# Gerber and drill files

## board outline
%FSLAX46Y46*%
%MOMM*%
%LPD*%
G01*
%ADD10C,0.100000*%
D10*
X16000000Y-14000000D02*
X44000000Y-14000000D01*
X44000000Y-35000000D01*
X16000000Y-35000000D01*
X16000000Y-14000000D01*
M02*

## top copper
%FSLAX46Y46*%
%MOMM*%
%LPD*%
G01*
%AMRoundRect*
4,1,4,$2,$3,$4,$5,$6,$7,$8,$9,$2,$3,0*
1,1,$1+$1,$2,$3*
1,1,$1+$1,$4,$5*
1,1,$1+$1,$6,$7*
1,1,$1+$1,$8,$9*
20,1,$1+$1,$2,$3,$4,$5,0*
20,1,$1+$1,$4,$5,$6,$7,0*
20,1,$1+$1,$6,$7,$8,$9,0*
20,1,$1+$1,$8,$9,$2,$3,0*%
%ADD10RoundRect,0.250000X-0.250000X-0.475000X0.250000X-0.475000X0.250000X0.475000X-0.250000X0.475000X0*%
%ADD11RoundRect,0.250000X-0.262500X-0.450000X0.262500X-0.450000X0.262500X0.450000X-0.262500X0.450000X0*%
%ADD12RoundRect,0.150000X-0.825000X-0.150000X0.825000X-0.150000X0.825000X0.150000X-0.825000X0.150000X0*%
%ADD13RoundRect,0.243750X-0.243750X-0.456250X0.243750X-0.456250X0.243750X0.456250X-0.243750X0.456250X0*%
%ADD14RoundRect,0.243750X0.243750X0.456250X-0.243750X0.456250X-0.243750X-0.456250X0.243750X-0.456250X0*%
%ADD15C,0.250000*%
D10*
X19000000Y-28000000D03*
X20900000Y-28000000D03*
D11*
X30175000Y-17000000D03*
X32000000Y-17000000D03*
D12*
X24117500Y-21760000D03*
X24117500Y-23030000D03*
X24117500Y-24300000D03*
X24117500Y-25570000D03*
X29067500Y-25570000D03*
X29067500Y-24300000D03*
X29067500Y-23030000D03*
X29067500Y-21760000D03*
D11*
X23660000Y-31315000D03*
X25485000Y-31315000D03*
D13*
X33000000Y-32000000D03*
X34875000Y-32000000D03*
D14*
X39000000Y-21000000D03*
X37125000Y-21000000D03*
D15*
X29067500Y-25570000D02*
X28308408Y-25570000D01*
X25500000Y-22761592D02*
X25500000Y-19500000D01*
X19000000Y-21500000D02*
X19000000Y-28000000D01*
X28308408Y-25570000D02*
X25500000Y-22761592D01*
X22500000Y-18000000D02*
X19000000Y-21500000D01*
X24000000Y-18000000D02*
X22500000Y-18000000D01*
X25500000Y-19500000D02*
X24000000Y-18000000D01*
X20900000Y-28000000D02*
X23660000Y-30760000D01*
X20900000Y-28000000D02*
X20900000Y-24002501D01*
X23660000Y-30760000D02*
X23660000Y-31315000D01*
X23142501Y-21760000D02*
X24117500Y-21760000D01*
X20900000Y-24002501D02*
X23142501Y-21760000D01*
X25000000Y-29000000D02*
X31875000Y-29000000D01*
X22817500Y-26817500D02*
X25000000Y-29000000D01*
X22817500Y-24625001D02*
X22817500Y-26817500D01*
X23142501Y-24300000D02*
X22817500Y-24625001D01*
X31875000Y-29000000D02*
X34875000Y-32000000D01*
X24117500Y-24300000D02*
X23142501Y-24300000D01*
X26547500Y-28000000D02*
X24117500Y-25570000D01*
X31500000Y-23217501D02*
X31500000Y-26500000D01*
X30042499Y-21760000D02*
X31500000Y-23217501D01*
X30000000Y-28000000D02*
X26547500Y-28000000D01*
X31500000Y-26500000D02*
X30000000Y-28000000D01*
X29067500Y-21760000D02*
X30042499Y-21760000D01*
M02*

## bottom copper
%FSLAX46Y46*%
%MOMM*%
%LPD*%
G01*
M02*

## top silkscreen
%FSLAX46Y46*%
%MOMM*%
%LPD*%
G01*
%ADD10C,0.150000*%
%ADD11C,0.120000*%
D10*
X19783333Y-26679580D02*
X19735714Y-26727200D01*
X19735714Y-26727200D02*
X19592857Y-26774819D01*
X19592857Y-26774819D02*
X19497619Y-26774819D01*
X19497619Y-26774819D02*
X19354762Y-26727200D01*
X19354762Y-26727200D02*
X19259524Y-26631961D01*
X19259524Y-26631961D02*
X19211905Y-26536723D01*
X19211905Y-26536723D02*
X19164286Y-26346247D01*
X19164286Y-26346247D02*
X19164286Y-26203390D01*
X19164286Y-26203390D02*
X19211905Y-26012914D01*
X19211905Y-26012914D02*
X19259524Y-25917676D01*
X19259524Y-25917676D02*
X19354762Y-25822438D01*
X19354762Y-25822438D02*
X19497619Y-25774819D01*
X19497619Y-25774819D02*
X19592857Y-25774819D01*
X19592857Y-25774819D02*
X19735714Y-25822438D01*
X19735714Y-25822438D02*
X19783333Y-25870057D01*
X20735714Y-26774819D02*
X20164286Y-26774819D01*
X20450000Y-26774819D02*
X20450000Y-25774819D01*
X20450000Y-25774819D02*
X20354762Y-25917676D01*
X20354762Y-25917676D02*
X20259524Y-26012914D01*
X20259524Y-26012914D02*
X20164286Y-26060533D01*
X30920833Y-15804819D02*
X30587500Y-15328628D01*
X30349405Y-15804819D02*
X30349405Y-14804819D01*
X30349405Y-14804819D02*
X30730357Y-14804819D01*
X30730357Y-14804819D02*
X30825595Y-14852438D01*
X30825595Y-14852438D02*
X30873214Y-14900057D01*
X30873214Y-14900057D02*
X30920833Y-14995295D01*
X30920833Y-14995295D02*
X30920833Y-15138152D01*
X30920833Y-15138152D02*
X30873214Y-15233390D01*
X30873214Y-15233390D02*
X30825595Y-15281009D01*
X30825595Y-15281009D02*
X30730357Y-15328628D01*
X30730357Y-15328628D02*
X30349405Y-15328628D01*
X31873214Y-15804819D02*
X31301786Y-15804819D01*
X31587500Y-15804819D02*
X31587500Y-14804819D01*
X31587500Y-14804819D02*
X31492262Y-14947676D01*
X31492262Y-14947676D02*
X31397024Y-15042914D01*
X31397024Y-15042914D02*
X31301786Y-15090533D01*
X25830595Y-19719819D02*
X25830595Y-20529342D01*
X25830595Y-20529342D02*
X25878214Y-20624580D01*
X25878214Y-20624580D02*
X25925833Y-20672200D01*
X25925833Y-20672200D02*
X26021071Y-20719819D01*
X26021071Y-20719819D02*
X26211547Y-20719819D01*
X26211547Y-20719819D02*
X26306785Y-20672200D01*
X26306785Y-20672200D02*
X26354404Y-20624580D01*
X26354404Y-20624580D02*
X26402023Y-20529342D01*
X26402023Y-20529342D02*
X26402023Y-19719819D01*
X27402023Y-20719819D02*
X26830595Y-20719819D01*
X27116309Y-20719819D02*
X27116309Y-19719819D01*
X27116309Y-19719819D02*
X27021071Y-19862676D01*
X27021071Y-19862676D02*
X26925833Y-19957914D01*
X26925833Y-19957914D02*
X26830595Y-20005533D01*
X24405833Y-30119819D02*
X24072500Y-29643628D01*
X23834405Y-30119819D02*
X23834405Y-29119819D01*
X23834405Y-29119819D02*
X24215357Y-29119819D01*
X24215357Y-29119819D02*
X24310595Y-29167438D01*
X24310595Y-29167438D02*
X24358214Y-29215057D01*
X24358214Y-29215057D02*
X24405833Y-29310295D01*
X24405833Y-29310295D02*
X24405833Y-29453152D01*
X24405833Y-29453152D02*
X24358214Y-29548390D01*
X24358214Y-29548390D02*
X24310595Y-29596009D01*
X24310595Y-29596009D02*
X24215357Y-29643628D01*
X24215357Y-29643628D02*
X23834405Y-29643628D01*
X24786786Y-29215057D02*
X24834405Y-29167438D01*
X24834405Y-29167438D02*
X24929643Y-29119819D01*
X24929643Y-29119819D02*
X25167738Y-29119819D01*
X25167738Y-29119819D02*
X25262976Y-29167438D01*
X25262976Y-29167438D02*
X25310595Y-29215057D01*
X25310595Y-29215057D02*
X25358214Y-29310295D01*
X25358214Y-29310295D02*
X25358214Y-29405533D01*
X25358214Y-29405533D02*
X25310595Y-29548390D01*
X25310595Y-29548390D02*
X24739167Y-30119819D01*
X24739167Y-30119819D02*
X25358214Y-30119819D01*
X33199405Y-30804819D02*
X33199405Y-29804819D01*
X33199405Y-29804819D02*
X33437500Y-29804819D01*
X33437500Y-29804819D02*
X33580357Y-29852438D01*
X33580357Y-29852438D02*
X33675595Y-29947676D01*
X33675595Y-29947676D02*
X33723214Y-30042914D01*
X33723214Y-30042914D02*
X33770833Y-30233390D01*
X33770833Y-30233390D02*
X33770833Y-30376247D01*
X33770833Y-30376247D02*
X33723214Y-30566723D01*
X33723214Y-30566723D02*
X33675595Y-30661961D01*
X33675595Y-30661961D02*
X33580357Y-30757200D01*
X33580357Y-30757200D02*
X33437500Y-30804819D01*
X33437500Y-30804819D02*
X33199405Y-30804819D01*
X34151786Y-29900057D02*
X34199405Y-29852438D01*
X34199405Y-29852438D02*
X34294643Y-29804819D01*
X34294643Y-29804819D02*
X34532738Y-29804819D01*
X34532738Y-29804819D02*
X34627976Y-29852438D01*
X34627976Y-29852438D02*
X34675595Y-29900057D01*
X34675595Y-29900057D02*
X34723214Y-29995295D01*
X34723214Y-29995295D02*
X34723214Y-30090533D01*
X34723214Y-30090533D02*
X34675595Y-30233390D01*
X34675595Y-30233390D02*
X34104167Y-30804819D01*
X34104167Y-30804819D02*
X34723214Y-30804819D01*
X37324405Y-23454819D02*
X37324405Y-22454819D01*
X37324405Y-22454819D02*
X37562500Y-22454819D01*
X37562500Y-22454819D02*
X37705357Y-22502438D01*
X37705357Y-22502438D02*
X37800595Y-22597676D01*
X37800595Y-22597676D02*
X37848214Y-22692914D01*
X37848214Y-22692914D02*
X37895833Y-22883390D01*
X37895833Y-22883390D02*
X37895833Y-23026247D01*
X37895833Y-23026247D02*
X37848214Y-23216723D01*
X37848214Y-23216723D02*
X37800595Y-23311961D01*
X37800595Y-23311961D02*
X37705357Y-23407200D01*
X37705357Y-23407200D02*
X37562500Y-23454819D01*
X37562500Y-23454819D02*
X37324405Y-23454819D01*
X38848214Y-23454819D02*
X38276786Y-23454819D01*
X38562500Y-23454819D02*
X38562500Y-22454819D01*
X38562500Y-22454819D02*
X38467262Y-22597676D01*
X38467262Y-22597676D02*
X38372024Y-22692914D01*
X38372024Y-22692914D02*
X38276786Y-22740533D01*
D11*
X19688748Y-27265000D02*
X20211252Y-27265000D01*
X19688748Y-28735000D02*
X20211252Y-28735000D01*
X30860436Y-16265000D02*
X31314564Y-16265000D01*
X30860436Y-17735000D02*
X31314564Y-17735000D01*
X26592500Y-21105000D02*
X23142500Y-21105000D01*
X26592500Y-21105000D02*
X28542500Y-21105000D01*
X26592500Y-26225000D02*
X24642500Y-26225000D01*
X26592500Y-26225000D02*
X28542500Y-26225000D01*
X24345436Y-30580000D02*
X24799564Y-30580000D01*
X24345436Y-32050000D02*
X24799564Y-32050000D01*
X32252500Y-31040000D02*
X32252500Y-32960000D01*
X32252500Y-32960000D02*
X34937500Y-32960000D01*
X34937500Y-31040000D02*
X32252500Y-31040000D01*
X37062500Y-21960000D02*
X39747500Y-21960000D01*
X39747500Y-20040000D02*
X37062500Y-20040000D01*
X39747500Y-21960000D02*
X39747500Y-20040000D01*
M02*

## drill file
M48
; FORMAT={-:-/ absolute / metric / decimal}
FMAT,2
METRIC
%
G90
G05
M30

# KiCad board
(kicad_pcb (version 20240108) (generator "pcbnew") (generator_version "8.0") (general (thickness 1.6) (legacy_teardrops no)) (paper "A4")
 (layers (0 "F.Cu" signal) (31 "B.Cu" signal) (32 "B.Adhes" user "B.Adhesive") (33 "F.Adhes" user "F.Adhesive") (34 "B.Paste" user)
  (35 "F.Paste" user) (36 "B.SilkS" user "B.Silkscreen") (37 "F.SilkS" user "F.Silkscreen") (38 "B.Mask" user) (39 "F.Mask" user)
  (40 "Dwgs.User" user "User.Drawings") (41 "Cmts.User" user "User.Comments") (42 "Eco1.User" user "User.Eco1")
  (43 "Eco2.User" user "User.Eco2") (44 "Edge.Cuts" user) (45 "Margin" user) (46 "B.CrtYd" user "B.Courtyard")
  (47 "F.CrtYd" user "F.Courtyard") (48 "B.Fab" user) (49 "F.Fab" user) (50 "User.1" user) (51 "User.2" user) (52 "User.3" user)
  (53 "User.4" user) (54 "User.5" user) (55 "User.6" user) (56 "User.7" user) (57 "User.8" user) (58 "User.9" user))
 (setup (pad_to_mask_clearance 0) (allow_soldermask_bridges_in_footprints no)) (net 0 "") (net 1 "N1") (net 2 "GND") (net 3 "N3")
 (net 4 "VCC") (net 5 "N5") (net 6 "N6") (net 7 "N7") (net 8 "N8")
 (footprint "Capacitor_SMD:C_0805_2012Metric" (layer "F.Cu") (at 19.95 28)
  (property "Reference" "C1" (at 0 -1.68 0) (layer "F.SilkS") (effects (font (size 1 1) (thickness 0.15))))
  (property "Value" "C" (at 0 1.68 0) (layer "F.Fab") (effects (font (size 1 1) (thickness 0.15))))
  (fp_line (start -0.261252 -0.735) (end 0.261252 -0.735) (stroke (width 0.12) (type solid)) (layer "F.SilkS"))
  (fp_line (start -0.261252 0.735) (end 0.261252 0.735) (stroke (width 0.12) (type solid)) (layer "F.SilkS"))
  (pad "1" smd roundrect (at -0.95 0) (size 1 1.45) (layers "F.Cu" "F.Paste" "F.Mask") (roundrect_rratio 0.25) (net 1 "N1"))
  (pad "2" smd roundrect (at 0.95 0) (size 1 1.45) (layers "F.Cu" "F.Paste" "F.Mask") (roundrect_rratio 0.25) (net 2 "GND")))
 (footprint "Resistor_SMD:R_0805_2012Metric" (layer "F.Cu") (at 31.0875 17)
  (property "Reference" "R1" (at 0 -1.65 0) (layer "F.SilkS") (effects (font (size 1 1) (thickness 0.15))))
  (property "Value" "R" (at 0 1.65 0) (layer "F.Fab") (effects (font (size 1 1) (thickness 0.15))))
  (fp_line (start -0.227064 -0.735) (end 0.227064 -0.735) (stroke (width 0.12) (type solid)) (layer "F.SilkS"))
  (fp_line (start -0.227064 0.735) (end 0.227064 0.735) (stroke (width 0.12) (type solid)) (layer "F.SilkS"))
  (pad "1" smd roundrect (at -0.9125 0) (size 1.025 1.4) (layers "F.Cu" "F.Paste" "F.Mask") (roundrect_rratio 0.243902) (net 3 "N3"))
  (pad "2" smd roundrect (at 0.9125 0) (size 1.025 1.4) (layers "F.Cu" "F.Paste" "F.Mask") (roundrect_rratio 0.243902) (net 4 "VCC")))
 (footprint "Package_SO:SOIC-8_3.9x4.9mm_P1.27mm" (layer "F.Cu") (at 26.5925 23.665)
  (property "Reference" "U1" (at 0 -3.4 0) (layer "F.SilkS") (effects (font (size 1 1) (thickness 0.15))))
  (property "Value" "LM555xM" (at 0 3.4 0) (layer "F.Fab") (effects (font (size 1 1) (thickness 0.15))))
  (fp_line (start 0 -2.56) (end -3.45 -2.56) (stroke (width 0.12) (type solid)) (layer "F.SilkS"))
  (fp_line (start 0 -2.56) (end 1.95 -2.56) (stroke (width 0.12) (type solid)) (layer "F.SilkS"))
  (fp_line (start 0 2.56) (end -1.95 2.56) (stroke (width 0.12) (type solid)) (layer "F.SilkS"))
  (fp_line (start 0 2.56) (end 1.95 2.56) (stroke (width 0.12) (type solid)) (layer "F.SilkS"))
  (pad "1" smd roundrect (at -2.475 -1.905) (size 1.95 0.6) (layers "F.Cu" "F.Paste" "F.Mask") (roundrect_rratio 0.25) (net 2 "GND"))
  (pad "2" smd roundrect (at -2.475 -0.635) (size 1.95 0.6) (layers "F.Cu" "F.Paste" "F.Mask") (roundrect_rratio 0.25) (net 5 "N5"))
  (pad "3" smd roundrect (at -2.475 0.635) (size 1.95 0.6) (layers "F.Cu" "F.Paste" "F.Mask") (roundrect_rratio 0.25) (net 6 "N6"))
  (pad "4" smd roundrect (at -2.475 1.905) (size 1.95 0.6) (layers "F.Cu" "F.Paste" "F.Mask") (roundrect_rratio 0.25) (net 4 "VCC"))
  (pad "5" smd roundrect (at 2.475 1.905) (size 1.95 0.6) (layers "F.Cu" "F.Paste" "F.Mask") (roundrect_rratio 0.25) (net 1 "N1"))
  (pad "6" smd roundrect (at 2.475 0.635) (size 1.95 0.6) (layers "F.Cu" "F.Paste" "F.Mask") (roundrect_rratio 0.25) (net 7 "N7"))
  (pad "7" smd roundrect (at 2.475 -0.635) (size 1.95 0.6) (layers "F.Cu" "F.Paste" "F.Mask") (roundrect_rratio 0.25) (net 7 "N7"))
  (pad "8" smd roundrect (at 2.475 -1.905) (size 1.95 0.6) (layers "F.Cu" "F.Paste" "F.Mask") (roundrect_rratio 0.25) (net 4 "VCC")))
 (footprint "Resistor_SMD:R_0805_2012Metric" (layer "F.Cu") (at 24.5725 31.315)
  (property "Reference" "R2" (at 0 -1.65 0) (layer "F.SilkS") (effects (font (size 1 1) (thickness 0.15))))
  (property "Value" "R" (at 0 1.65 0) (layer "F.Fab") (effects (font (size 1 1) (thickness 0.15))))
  (fp_line (start -0.227064 -0.735) (end 0.227064 -0.735) (stroke (width 0.12) (type solid)) (layer "F.SilkS"))
  (fp_line (start -0.227064 0.735) (end 0.227064 0.735) (stroke (width 0.12) (type solid)) (layer "F.SilkS"))
  (pad "1" smd roundrect (at -0.9125 0) (size 1.025 1.4) (layers "F.Cu" "F.Paste" "F.Mask") (roundrect_rratio 0.243902) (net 2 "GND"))
  (pad "2" smd roundrect (at 0.9125 0) (size 1.025 1.4) (layers "F.Cu" "F.Paste" "F.Mask") (roundrect_rratio 0.243902) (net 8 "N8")))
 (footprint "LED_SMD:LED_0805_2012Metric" (layer "F.Cu") (at 33.9375 32)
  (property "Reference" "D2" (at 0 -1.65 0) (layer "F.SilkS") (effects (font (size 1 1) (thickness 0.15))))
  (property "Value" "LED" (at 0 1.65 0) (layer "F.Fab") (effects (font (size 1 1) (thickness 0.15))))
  (fp_line (start -1.685 -0.96) (end -1.685 0.96) (stroke (width 0.12) (type solid)) (layer "F.SilkS"))
  (fp_line (start -1.685 0.96) (end 1 0.96) (stroke (width 0.12) (type solid)) (layer "F.SilkS"))
  (fp_line (start 1 -0.96) (end -1.685 -0.96) (stroke (width 0.12) (type solid)) (layer "F.SilkS"))
  (pad "1" smd roundrect (at -0.9375 0) (size 0.975 1.4) (layers "F.Cu" "F.Paste" "F.Mask") (roundrect_rratio 0.25) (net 8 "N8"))
  (pad "2" smd roundrect (at 0.9375 0) (size 0.975 1.4) (layers "F.Cu" "F.Paste" "F.Mask") (roundrect_rratio 0.25) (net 6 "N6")))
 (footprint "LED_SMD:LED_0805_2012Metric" (layer "F.Cu") (at 38.0625 21 180)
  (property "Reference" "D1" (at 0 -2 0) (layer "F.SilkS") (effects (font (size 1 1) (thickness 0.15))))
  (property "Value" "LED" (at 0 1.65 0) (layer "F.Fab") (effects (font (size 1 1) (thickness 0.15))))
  (fp_line (start 1 -0.96) (end -1.685 -0.96) (stroke (width 0.12) (type solid)) (layer "F.SilkS"))
  (fp_line (start -1.685 0.96) (end 1 0.96) (stroke (width 0.12) (type solid)) (layer "F.SilkS"))
  (fp_line (start -1.685 -0.96) (end -1.685 0.96) (stroke (width 0.12) (type solid)) (layer "F.SilkS"))
  (pad "1" smd roundrect (at -0.9375 0 180) (size 0.975 1.4) (layers "F.Cu" "F.Paste" "F.Mask") (roundrect_rratio 0.25) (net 6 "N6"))
  (pad "2" smd roundrect (at 0.9375 0 180) (size 0.975 1.4) (layers "F.Cu" "F.Paste" "F.Mask") (roundrect_rratio 0.25) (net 3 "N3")))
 (gr_rect (start 16 14) (end 44 35) (stroke (width 0.1) (type default)) (fill none) (layer "Edge.Cuts"))
 (segment (start 29.0675 25.57) (end 28.308408 25.57) (width 0.25) (layer "F.Cu") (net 1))
 (segment (start 25.5 22.761592) (end 25.5 19.5) (width 0.25) (layer "F.Cu") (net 1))
 (segment (start 19 21.5) (end 19 28) (width 0.25) (layer "F.Cu") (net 1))
 (segment (start 28.308408 25.57) (end 25.5 22.761592) (width 0.25) (layer "F.Cu") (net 1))
 (segment (start 22.5 18) (end 19 21.5) (width 0.25) (layer "F.Cu") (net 1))
 (segment (start 24 18) (end 22.5 18) (width 0.25) (layer "F.Cu") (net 1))
 (segment (start 25.5 19.5) (end 24 18) (width 0.25) (layer "F.Cu") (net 1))
 (segment (start 20.9 28) (end 23.66 30.76) (width 0.25) (layer "F.Cu") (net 2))
 (segment (start 20.9 28) (end 20.9 24.002501) (width 0.25) (layer "F.Cu") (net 2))
 (segment (start 23.66 30.76) (end 23.66 31.315) (width 0.25) (layer "F.Cu") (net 2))
 (segment (start 23.142501 21.76) (end 24.1175 21.76) (width 0.25) (layer "F.Cu") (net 2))
 (segment (start 20.9 24.002501) (end 23.142501 21.76) (width 0.25) (layer "F.Cu") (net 2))
 (segment (start 25 29) (end 31.875 29) (width 0.25) (layer "F.Cu") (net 6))
 (segment (start 22.8175 26.8175) (end 25 29) (width 0.25) (layer "F.Cu") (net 6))
 (segment (start 22.8175 24.625001) (end 22.8175 26.8175) (width 0.25) (layer "F.Cu") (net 6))
 (segment (start 23.142501 24.3) (end 22.8175 24.625001) (width 0.25) (layer "F.Cu") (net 6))
 (segment (start 31.875 29) (end 34.875 32) (width 0.25) (layer "F.Cu") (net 6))
 (segment (start 24.1175 24.3) (end 23.142501 24.3) (width 0.25) (layer "F.Cu") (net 6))
 (segment (start 26.5475 28) (end 24.1175 25.57) (width 0.25) (layer "F.Cu") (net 4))
 (segment (start 31.5 23.217501) (end 31.5 26.5) (width 0.25) (layer "F.Cu") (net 4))
 (segment (start 30.042499 21.76) (end 31.5 23.217501) (width 0.25) (layer "F.Cu") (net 4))
 (segment (start 30 28) (end 26.5475 28) (width 0.25) (layer "F.Cu") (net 4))
 (segment (start 31.5 26.5) (end 30 28) (width 0.25) (layer "F.Cu") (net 4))
 (segment (start 29.0675 21.76) (end 30.042499 21.76) (width 0.25) (layer "F.Cu") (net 4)))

